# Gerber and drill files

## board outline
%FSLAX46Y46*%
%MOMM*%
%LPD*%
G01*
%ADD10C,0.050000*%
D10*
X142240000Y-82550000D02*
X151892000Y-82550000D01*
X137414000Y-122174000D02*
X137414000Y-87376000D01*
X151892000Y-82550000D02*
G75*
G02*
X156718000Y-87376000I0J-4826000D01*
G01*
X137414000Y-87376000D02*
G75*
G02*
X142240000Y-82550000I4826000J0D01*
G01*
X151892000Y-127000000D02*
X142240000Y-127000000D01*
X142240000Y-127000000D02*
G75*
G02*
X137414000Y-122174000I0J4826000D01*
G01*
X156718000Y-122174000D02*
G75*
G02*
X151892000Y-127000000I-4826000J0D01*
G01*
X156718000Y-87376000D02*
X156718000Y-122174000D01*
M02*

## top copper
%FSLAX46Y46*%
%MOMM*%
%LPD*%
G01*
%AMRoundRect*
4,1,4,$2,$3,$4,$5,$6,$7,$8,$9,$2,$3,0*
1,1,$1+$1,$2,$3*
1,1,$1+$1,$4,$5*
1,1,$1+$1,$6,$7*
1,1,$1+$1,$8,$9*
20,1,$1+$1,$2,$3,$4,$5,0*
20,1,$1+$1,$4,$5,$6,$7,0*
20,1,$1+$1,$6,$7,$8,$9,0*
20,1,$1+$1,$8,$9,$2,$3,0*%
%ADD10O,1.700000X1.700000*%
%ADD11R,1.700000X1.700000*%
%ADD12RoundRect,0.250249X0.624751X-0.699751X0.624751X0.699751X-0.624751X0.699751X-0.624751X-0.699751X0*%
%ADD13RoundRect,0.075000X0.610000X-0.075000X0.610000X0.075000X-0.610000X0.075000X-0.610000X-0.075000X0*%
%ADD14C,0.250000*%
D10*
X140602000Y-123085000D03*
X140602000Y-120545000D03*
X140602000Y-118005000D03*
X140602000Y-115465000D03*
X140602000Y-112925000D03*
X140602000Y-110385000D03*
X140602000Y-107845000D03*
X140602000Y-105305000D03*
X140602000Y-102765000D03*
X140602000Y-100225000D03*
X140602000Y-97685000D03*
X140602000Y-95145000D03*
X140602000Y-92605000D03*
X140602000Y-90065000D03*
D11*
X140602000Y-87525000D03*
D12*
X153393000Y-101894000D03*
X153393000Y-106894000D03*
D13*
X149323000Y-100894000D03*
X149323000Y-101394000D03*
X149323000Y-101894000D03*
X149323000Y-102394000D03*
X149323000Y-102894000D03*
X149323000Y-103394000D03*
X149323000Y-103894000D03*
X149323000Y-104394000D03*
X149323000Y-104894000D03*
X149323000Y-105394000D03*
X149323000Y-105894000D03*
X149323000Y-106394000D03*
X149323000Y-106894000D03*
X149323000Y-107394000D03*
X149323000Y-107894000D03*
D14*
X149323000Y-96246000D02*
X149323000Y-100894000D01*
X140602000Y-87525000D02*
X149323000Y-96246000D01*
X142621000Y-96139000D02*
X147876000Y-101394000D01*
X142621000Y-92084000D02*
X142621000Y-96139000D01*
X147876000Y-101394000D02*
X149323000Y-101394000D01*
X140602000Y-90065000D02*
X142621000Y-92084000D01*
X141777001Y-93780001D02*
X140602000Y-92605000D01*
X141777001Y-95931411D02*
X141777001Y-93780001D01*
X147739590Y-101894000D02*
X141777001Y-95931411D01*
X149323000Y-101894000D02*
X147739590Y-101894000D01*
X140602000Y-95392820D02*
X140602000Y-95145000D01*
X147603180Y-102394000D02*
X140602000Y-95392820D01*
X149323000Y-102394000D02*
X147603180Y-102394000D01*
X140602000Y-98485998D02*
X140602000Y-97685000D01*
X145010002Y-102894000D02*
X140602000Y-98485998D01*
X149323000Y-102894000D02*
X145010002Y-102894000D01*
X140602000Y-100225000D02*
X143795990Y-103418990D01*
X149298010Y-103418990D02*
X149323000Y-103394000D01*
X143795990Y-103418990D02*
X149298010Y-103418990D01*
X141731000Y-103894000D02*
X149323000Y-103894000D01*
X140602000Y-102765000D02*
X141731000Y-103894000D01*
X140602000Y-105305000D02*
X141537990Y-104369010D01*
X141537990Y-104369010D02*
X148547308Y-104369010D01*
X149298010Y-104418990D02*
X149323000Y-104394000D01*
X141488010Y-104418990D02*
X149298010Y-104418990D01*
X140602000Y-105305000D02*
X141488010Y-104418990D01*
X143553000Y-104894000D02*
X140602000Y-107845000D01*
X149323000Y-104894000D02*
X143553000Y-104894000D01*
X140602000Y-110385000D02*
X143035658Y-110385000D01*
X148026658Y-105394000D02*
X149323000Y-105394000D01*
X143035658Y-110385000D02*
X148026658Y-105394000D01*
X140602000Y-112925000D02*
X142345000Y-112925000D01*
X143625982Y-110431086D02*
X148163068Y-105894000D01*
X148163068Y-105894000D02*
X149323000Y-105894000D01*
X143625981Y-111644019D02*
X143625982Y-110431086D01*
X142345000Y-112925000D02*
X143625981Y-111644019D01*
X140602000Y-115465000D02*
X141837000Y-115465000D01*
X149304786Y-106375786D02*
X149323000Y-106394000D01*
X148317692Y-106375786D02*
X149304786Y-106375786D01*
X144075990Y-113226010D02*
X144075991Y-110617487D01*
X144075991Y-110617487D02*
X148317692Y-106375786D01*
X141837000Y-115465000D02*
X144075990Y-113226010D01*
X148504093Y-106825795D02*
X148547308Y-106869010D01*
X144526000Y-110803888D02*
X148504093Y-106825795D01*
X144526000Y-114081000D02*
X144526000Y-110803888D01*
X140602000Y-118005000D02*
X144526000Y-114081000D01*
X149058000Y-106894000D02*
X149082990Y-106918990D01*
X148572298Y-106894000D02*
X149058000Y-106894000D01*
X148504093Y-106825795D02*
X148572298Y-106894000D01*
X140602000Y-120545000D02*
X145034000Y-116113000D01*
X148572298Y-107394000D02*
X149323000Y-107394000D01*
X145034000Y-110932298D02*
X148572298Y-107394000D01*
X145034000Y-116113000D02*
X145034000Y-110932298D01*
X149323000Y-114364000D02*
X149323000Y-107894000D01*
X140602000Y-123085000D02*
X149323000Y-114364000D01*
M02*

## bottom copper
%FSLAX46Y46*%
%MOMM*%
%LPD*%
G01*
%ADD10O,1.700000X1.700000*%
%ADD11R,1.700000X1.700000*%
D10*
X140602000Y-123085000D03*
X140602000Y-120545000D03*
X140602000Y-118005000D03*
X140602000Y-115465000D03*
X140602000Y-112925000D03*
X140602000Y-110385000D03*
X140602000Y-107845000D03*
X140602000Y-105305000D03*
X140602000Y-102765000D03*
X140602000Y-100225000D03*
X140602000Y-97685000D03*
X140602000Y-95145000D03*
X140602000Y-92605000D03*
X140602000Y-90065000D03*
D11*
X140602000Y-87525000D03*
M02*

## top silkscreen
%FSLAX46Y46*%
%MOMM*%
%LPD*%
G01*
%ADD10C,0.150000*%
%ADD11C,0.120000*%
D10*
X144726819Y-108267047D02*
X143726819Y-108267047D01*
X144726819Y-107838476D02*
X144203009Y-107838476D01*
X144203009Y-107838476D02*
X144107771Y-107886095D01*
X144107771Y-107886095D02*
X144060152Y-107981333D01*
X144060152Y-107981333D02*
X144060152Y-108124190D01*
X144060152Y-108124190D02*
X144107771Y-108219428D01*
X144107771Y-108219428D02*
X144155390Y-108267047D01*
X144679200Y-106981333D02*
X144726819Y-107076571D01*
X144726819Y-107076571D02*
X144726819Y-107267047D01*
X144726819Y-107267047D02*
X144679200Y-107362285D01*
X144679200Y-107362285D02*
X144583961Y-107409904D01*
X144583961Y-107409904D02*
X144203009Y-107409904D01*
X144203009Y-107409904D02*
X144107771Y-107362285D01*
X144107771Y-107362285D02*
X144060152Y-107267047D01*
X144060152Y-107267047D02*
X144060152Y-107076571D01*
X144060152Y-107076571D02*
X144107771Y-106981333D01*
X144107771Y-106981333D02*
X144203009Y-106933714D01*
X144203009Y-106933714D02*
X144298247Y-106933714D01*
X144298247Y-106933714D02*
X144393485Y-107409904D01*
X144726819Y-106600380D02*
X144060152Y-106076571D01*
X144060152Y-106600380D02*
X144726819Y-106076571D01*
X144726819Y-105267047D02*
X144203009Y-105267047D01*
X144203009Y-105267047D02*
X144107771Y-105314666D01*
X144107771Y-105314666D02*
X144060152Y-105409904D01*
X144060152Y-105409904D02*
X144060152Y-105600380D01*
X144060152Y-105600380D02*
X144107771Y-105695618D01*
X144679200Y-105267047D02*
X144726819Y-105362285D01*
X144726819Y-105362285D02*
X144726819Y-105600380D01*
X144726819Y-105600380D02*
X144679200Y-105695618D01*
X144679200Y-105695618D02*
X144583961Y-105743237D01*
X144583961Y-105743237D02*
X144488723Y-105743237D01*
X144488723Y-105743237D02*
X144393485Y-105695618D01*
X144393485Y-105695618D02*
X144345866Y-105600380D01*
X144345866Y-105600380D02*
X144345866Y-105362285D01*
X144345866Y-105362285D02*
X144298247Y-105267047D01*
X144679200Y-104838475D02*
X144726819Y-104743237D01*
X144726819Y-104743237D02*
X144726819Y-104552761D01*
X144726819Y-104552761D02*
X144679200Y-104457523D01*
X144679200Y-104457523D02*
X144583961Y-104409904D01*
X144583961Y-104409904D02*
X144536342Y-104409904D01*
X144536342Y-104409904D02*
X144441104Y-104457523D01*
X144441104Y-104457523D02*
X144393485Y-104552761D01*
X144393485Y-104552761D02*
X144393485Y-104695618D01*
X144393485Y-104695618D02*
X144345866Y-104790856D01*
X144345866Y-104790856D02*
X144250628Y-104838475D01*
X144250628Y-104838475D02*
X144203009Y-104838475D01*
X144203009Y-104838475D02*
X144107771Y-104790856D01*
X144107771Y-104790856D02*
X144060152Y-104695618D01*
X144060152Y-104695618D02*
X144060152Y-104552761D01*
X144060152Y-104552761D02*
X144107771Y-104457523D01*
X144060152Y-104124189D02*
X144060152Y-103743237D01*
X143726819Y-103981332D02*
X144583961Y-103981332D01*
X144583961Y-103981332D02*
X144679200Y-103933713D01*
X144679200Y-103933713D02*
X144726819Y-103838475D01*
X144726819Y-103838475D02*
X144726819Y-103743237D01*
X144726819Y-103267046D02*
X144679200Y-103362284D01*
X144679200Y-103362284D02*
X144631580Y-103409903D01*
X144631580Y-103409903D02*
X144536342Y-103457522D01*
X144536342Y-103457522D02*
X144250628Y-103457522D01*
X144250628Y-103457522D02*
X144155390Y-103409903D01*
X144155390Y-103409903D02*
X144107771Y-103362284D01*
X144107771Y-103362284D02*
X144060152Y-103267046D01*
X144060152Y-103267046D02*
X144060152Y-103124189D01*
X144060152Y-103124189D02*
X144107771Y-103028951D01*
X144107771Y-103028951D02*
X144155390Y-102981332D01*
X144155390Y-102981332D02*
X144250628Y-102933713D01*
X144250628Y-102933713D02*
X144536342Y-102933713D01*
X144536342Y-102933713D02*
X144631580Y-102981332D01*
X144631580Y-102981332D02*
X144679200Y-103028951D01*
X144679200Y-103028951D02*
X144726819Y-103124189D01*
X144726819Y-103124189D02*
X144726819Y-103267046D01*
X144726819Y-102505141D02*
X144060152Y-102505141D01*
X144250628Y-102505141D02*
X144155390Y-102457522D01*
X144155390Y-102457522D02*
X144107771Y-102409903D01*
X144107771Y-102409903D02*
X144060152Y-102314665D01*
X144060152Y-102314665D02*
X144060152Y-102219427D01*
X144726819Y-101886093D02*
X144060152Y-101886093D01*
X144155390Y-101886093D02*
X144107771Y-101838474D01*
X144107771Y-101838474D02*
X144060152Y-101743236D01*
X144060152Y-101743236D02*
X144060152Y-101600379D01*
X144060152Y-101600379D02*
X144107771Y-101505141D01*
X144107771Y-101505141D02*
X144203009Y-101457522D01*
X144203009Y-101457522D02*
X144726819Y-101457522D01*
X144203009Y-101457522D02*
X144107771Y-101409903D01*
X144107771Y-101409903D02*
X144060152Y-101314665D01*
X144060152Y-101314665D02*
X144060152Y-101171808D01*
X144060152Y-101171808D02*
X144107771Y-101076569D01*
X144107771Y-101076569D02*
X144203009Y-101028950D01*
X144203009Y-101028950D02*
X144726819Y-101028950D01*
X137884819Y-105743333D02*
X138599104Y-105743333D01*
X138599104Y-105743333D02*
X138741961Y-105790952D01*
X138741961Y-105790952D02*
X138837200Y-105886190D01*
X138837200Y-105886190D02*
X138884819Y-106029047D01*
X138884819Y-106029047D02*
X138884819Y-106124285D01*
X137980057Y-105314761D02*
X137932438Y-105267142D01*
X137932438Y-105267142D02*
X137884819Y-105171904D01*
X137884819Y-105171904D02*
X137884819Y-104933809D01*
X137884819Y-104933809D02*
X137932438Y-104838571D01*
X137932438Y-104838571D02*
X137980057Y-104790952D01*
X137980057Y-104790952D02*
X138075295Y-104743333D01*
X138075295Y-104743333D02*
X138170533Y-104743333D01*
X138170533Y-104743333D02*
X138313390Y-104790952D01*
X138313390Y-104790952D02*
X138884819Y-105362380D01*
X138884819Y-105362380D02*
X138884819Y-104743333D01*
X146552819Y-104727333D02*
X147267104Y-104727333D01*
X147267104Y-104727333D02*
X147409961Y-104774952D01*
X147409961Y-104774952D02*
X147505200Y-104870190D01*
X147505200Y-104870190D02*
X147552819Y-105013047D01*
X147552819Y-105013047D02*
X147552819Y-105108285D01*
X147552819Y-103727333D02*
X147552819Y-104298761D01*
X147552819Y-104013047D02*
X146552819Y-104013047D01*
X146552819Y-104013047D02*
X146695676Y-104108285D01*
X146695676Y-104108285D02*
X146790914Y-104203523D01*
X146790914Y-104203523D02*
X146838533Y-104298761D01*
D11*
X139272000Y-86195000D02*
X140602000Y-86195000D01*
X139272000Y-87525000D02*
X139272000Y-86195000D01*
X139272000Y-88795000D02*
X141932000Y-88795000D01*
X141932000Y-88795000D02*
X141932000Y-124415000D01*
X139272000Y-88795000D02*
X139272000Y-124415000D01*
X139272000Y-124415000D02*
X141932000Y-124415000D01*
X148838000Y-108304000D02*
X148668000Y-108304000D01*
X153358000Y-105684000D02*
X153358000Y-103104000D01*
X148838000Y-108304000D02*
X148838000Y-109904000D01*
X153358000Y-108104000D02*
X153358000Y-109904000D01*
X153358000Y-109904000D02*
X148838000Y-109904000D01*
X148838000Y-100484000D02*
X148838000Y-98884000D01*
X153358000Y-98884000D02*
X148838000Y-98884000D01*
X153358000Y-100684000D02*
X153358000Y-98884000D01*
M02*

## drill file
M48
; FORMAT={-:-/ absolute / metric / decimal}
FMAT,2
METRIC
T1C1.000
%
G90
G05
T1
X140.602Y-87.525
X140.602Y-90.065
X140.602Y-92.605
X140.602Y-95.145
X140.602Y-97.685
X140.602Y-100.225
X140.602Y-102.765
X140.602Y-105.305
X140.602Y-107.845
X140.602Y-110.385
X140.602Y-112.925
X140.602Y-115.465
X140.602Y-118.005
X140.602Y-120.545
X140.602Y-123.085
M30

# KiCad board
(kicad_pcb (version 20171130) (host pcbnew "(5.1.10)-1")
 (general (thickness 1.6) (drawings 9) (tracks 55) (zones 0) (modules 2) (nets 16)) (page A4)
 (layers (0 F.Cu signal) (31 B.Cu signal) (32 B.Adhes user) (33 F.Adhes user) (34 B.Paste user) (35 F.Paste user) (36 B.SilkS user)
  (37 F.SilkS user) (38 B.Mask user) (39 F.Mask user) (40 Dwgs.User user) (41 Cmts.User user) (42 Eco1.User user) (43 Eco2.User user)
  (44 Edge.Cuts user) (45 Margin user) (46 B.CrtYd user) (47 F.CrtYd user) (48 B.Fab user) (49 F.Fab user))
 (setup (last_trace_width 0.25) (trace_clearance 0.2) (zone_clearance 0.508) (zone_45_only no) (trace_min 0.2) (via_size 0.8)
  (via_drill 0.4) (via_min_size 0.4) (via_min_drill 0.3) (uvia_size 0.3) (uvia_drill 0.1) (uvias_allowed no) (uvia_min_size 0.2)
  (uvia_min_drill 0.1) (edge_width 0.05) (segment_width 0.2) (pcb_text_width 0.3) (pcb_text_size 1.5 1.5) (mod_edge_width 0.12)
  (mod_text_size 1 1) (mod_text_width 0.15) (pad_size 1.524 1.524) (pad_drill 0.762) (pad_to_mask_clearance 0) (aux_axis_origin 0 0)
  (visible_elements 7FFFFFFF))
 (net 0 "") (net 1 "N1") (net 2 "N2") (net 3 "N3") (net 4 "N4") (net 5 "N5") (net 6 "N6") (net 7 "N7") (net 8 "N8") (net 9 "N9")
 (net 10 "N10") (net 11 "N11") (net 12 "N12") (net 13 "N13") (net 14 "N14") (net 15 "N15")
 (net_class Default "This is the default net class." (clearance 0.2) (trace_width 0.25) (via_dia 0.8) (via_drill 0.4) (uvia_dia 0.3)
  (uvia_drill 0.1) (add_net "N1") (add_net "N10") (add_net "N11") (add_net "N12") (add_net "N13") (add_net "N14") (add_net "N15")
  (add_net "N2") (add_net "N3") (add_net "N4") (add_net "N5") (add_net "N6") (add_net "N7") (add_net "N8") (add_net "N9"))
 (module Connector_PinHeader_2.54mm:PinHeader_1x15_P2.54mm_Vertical (layer F.Cu) (at 140.602 87.525)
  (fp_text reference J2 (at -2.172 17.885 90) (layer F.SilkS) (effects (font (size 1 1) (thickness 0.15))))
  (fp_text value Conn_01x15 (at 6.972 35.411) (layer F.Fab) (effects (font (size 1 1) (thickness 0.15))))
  (fp_line (start -1.33 -1.33) (end 0 -1.33) (layer F.SilkS) (width 0.12))
  (fp_line (start -1.33 0) (end -1.33 -1.33) (layer F.SilkS) (width 0.12))
  (fp_line (start -1.33 1.27) (end 1.33 1.27) (layer F.SilkS) (width 0.12))
  (fp_line (start 1.33 1.27) (end 1.33 36.89) (layer F.SilkS) (width 0.12))
  (fp_line (start -1.33 1.27) (end -1.33 36.89) (layer F.SilkS) (width 0.12))
  (fp_line (start -1.33 36.89) (end 1.33 36.89) (layer F.SilkS) (width 0.12))
  (pad 15 thru_hole oval (at 0 35.56) (size 1.7 1.7) (drill 1) (layers *.Cu *.Mask) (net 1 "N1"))
  (pad 14 thru_hole oval (at 0 33.02) (size 1.7 1.7) (drill 1) (layers *.Cu *.Mask) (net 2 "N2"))
  (pad 13 thru_hole oval (at 0 30.48) (size 1.7 1.7) (drill 1) (layers *.Cu *.Mask) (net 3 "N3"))
  (pad 12 thru_hole oval (at 0 27.94) (size 1.7 1.7) (drill 1) (layers *.Cu *.Mask) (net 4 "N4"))
  (pad 11 thru_hole oval (at 0 25.4) (size 1.7 1.7) (drill 1) (layers *.Cu *.Mask) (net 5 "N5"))
  (pad 10 thru_hole oval (at 0 22.86) (size 1.7 1.7) (drill 1) (layers *.Cu *.Mask) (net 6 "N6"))
  (pad 9 thru_hole oval (at 0 20.32) (size 1.7 1.7) (drill 1) (layers *.Cu *.Mask) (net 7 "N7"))
  (pad 8 thru_hole oval (at 0 17.78) (size 1.7 1.7) (drill 1) (layers *.Cu *.Mask) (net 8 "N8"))
  (pad 7 thru_hole oval (at 0 15.24) (size 1.7 1.7) (drill 1) (layers *.Cu *.Mask) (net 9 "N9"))
  (pad 6 thru_hole oval (at 0 12.7) (size 1.7 1.7) (drill 1) (layers *.Cu *.Mask) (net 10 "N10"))
  (pad 5 thru_hole oval (at 0 10.16) (size 1.7 1.7) (drill 1) (layers *.Cu *.Mask) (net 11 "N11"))
  (pad 4 thru_hole oval (at 0 7.62) (size 1.7 1.7) (drill 1) (layers *.Cu *.Mask) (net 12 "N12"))
  (pad 3 thru_hole oval (at 0 5.08) (size 1.7 1.7) (drill 1) (layers *.Cu *.Mask) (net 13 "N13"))
  (pad 2 thru_hole oval (at 0 2.54) (size 1.7 1.7) (drill 1) (layers *.Cu *.Mask) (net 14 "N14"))
  (pad 1 thru_hole rect (at 0 0) (size 1.7 1.7) (drill 1) (layers *.Cu *.Mask) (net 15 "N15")))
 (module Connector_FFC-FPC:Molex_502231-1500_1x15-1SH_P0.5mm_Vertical (layer F.Cu) (at 150.368 104.394 90)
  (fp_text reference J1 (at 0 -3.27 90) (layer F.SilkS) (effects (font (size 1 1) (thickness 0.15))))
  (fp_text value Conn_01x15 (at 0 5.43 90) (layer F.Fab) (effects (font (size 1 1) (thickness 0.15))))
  (fp_line (start -3.91 -1.53) (end -3.91 -1.7) (layer F.SilkS) (width 0.12))
  (fp_line (start -1.29 2.99) (end 1.29 2.99) (layer F.SilkS) (width 0.12))
  (fp_line (start -3.91 -1.53) (end -5.51 -1.53) (layer F.SilkS) (width 0.12))
  (fp_line (start -3.71 2.99) (end -5.51 2.99) (layer F.SilkS) (width 0.12))
  (fp_line (start -5.51 2.99) (end -5.51 -1.53) (layer F.SilkS) (width 0.12))
  (fp_line (start 3.91 -1.53) (end 5.51 -1.53) (layer F.SilkS) (width 0.12))
  (fp_line (start 5.51 2.99) (end 5.51 -1.53) (layer F.SilkS) (width 0.12))
  (fp_line (start 3.71 2.99) (end 5.51 2.99) (layer F.SilkS) (width 0.12))
  (pad SH smd roundrect (at 2.5 3.025 90) (size 1.9 1.75) (layers F.Cu F.Paste F.Mask) (roundrect_rratio 0.1429994285714286))
  (pad SH smd roundrect (at -2.5 3.025 90) (size 1.9 1.75) (layers F.Cu F.Paste F.Mask) (roundrect_rratio 0.1429994285714286))
  (pad 15 smd roundrect (at 3.5 -1.045 90) (size 0.3 1.37) (layers F.Cu F.Paste F.Mask) (roundrect_rratio 0.25) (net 15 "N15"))
  (pad 14 smd roundrect (at 3 -1.045 90) (size 0.3 1.37) (layers F.Cu F.Paste F.Mask) (roundrect_rratio 0.25) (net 14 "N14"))
  (pad 13 smd roundrect (at 2.5 -1.045 90) (size 0.3 1.37) (layers F.Cu F.Paste F.Mask) (roundrect_rratio 0.25) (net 13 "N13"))
  (pad 12 smd roundrect (at 2 -1.045 90) (size 0.3 1.37) (layers F.Cu F.Paste F.Mask) (roundrect_rratio 0.25) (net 12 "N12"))
  (pad 11 smd roundrect (at 1.5 -1.045 90) (size 0.3 1.37) (layers F.Cu F.Paste F.Mask) (roundrect_rratio 0.25) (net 11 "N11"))
  (pad 10 smd roundrect (at 1 -1.045 90) (size 0.3 1.37) (layers F.Cu F.Paste F.Mask) (roundrect_rratio 0.25) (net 10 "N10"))
  (pad 9 smd roundrect (at 0.5 -1.045 90) (size 0.3 1.37) (layers F.Cu F.Paste F.Mask) (roundrect_rratio 0.25) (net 9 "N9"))
  (pad 8 smd roundrect (at 0 -1.045 90) (size 0.3 1.37) (layers F.Cu F.Paste F.Mask) (roundrect_rratio 0.25) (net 8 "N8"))
  (pad 7 smd roundrect (at -0.5 -1.045 90) (size 0.3 1.37) (layers F.Cu F.Paste F.Mask) (roundrect_rratio 0.25) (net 7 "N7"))
  (pad 6 smd roundrect (at -1 -1.045 90) (size 0.3 1.37) (layers F.Cu F.Paste F.Mask) (roundrect_rratio 0.25) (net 6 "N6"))
  (pad 5 smd roundrect (at -1.5 -1.045 90) (size 0.3 1.37) (layers F.Cu F.Paste F.Mask) (roundrect_rratio 0.25) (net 5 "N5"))
  (pad 4 smd roundrect (at -2 -1.045 90) (size 0.3 1.37) (layers F.Cu F.Paste F.Mask) (roundrect_rratio 0.25) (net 4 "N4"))
  (pad 3 smd roundrect (at -2.5 -1.045 90) (size 0.3 1.37) (layers F.Cu F.Paste F.Mask) (roundrect_rratio 0.25) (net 3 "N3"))
  (pad 2 smd roundrect (at -3 -1.045 90) (size 0.3 1.37) (layers F.Cu F.Paste F.Mask) (roundrect_rratio 0.25) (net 2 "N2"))
  (pad 1 smd roundrect (at -3.5 -1.045 90) (size 0.3 1.37) (layers F.Cu F.Paste F.Mask) (roundrect_rratio 0.25) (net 1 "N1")))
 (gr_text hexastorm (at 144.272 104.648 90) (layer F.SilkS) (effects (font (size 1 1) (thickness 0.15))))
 (gr_line (start 142.24 82.55) (end 151.892 82.55) (layer Edge.Cuts) (width 0.05))
 (gr_line (start 137.414 122.174) (end 137.414 87.376) (layer Edge.Cuts) (width 0.05))
 (gr_arc (start 151.892 87.376) (end 156.718 87.376) (angle -90) (layer Edge.Cuts) (width 0.05))
 (gr_arc (start 142.24 87.376) (end 142.24 82.55) (angle -90) (layer Edge.Cuts) (width 0.05))
 (gr_line (start 151.892 127) (end 142.24 127) (layer Edge.Cuts) (width 0.05))
 (gr_arc (start 142.24 122.174) (end 137.414 122.174) (angle -90) (layer Edge.Cuts) (width 0.05))
 (gr_arc (start 151.892 122.174) (end 151.892 127) (angle -90) (layer Edge.Cuts) (width 0.05))
 (gr_line (start 156.718 87.376) (end 156.718 122.174) (layer Edge.Cuts) (width 0.05))
 (segment (start 149.323 96.246) (end 149.323 100.894) (width 0.25) (layer F.Cu) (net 15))
 (segment (start 140.602 87.525) (end 149.323 96.246) (width 0.25) (layer F.Cu) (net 15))
 (segment (start 142.621 96.139) (end 147.876 101.394) (width 0.25) (layer F.Cu) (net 14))
 (segment (start 142.621 92.084) (end 142.621 96.139) (width 0.25) (layer F.Cu) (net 14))
 (segment (start 147.876 101.394) (end 149.323 101.394) (width 0.25) (layer F.Cu) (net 14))
 (segment (start 140.602 90.065) (end 142.621 92.084) (width 0.25) (layer F.Cu) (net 14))
 (segment (start 141.777001 93.780001) (end 140.602 92.605) (width 0.25) (layer F.Cu) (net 13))
 (segment (start 141.777001 95.931411) (end 141.777001 93.780001) (width 0.25) (layer F.Cu) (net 13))
 (segment (start 147.73959 101.894) (end 141.777001 95.931411) (width 0.25) (layer F.Cu) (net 13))
 (segment (start 149.323 101.894) (end 147.73959 101.894) (width 0.25) (layer F.Cu) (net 13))
 (segment (start 140.602 95.39282) (end 140.602 95.145) (width 0.25) (layer F.Cu) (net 12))
 (segment (start 147.60318 102.394) (end 140.602 95.39282) (width 0.25) (layer F.Cu) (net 12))
 (segment (start 149.323 102.394) (end 147.60318 102.394) (width 0.25) (layer F.Cu) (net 12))
 (segment (start 140.602 98.485998) (end 140.602 97.685) (width 0.25) (layer F.Cu) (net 11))
 (segment (start 145.010002 102.894) (end 140.602 98.485998) (width 0.25) (layer F.Cu) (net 11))
 (segment (start 149.323 102.894) (end 145.010002 102.894) (width 0.25) (layer F.Cu) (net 11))
 (segment (start 140.602 100.225) (end 143.79599 103.41899) (width 0.25) (layer F.Cu) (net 10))
 (segment (start 149.29801 103.41899) (end 149.323 103.394) (width 0.25) (layer F.Cu) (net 10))
 (segment (start 143.79599 103.41899) (end 149.29801 103.41899) (width 0.25) (layer F.Cu) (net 10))
 (segment (start 141.731 103.894) (end 149.323 103.894) (width 0.25) (layer F.Cu) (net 9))
 (segment (start 140.602 102.765) (end 141.731 103.894) (width 0.25) (layer F.Cu) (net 9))
 (segment (start 140.602 105.305) (end 141.53799 104.36901) (width 0.25) (layer F.Cu) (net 8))
 (segment (start 141.53799 104.36901) (end 148.547308 104.36901) (width 0.25) (layer F.Cu) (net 8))
 (segment (start 149.29801 104.41899) (end 149.323 104.394) (width 0.25) (layer F.Cu) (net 8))
 (segment (start 141.48801 104.41899) (end 149.29801 104.41899) (width 0.25) (layer F.Cu) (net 8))
 (segment (start 140.602 105.305) (end 141.48801 104.41899) (width 0.25) (layer F.Cu) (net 8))
 (segment (start 143.553 104.894) (end 140.602 107.845) (width 0.25) (layer F.Cu) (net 7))
 (segment (start 149.323 104.894) (end 143.553 104.894) (width 0.25) (layer F.Cu) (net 7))
 (segment (start 140.602 110.385) (end 143.035658 110.385) (width 0.25) (layer F.Cu) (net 6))
 (segment (start 148.026658 105.394) (end 149.323 105.394) (width 0.25) (layer F.Cu) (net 6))
 (segment (start 143.035658 110.385) (end 148.026658 105.394) (width 0.25) (layer F.Cu) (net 6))
 (segment (start 140.602 112.925) (end 142.345 112.925) (width 0.25) (layer F.Cu) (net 5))
 (segment (start 143.625982 110.431086) (end 148.163068 105.894) (width 0.25) (layer F.Cu) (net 5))
 (segment (start 148.163068 105.894) (end 149.323 105.894) (width 0.25) (layer F.Cu) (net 5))
 (segment (start 143.625981 111.644019) (end 143.625982 110.431086) (width 0.25) (layer F.Cu) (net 5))
 (segment (start 142.345 112.925) (end 143.625981 111.644019) (width 0.25) (layer F.Cu) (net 5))
 (segment (start 140.602 115.465) (end 141.837 115.465) (width 0.25) (layer F.Cu) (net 4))
 (segment (start 149.304786 106.375786) (end 149.323 106.394) (width 0.25) (layer F.Cu) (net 4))
 (segment (start 148.317692 106.375786) (end 149.304786 106.375786) (width 0.25) (layer F.Cu) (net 4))
 (segment (start 144.07599 113.22601) (end 144.075991 110.617487) (width 0.25) (layer F.Cu) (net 4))
 (segment (start 144.075991 110.617487) (end 148.317692 106.375786) (width 0.25) (layer F.Cu) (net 4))
 (segment (start 141.837 115.465) (end 144.07599 113.22601) (width 0.25) (layer F.Cu) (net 4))
 (segment (start 148.504093 106.825795) (end 148.547308 106.86901) (width 0.25) (layer F.Cu) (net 3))
 (segment (start 144.526 110.803888) (end 148.504093 106.825795) (width 0.25) (layer F.Cu) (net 3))
 (segment (start 144.526 114.081) (end 144.526 110.803888) (width 0.25) (layer F.Cu) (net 3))
 (segment (start 140.602 118.005) (end 144.526 114.081) (width 0.25) (layer F.Cu) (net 3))
 (segment (start 149.058 106.894) (end 149.08299 106.91899) (width 0.25) (layer F.Cu) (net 3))
 (segment (start 148.572298 106.894) (end 149.058 106.894) (width 0.25) (layer F.Cu) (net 3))
 (segment (start 148.504093 106.825795) (end 148.572298 106.894) (width 0.25) (layer F.Cu) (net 3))
 (segment (start 140.602 120.545) (end 145.034 116.113) (width 0.25) (layer F.Cu) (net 2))
 (segment (start 148.572298 107.394) (end 149.323 107.394) (width 0.25) (layer F.Cu) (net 2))
 (segment (start 145.034 110.932298) (end 148.572298 107.394) (width 0.25) (layer F.Cu) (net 2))
 (segment (start 145.034 116.113) (end 145.034 110.932298) (width 0.25) (layer F.Cu) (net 2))
 (segment (start 149.323 114.364) (end 149.323 107.894) (width 0.25) (layer F.Cu) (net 1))
 (segment (start 140.602 123.085) (end 149.323 114.364) (width 0.25) (layer F.Cu) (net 1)))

